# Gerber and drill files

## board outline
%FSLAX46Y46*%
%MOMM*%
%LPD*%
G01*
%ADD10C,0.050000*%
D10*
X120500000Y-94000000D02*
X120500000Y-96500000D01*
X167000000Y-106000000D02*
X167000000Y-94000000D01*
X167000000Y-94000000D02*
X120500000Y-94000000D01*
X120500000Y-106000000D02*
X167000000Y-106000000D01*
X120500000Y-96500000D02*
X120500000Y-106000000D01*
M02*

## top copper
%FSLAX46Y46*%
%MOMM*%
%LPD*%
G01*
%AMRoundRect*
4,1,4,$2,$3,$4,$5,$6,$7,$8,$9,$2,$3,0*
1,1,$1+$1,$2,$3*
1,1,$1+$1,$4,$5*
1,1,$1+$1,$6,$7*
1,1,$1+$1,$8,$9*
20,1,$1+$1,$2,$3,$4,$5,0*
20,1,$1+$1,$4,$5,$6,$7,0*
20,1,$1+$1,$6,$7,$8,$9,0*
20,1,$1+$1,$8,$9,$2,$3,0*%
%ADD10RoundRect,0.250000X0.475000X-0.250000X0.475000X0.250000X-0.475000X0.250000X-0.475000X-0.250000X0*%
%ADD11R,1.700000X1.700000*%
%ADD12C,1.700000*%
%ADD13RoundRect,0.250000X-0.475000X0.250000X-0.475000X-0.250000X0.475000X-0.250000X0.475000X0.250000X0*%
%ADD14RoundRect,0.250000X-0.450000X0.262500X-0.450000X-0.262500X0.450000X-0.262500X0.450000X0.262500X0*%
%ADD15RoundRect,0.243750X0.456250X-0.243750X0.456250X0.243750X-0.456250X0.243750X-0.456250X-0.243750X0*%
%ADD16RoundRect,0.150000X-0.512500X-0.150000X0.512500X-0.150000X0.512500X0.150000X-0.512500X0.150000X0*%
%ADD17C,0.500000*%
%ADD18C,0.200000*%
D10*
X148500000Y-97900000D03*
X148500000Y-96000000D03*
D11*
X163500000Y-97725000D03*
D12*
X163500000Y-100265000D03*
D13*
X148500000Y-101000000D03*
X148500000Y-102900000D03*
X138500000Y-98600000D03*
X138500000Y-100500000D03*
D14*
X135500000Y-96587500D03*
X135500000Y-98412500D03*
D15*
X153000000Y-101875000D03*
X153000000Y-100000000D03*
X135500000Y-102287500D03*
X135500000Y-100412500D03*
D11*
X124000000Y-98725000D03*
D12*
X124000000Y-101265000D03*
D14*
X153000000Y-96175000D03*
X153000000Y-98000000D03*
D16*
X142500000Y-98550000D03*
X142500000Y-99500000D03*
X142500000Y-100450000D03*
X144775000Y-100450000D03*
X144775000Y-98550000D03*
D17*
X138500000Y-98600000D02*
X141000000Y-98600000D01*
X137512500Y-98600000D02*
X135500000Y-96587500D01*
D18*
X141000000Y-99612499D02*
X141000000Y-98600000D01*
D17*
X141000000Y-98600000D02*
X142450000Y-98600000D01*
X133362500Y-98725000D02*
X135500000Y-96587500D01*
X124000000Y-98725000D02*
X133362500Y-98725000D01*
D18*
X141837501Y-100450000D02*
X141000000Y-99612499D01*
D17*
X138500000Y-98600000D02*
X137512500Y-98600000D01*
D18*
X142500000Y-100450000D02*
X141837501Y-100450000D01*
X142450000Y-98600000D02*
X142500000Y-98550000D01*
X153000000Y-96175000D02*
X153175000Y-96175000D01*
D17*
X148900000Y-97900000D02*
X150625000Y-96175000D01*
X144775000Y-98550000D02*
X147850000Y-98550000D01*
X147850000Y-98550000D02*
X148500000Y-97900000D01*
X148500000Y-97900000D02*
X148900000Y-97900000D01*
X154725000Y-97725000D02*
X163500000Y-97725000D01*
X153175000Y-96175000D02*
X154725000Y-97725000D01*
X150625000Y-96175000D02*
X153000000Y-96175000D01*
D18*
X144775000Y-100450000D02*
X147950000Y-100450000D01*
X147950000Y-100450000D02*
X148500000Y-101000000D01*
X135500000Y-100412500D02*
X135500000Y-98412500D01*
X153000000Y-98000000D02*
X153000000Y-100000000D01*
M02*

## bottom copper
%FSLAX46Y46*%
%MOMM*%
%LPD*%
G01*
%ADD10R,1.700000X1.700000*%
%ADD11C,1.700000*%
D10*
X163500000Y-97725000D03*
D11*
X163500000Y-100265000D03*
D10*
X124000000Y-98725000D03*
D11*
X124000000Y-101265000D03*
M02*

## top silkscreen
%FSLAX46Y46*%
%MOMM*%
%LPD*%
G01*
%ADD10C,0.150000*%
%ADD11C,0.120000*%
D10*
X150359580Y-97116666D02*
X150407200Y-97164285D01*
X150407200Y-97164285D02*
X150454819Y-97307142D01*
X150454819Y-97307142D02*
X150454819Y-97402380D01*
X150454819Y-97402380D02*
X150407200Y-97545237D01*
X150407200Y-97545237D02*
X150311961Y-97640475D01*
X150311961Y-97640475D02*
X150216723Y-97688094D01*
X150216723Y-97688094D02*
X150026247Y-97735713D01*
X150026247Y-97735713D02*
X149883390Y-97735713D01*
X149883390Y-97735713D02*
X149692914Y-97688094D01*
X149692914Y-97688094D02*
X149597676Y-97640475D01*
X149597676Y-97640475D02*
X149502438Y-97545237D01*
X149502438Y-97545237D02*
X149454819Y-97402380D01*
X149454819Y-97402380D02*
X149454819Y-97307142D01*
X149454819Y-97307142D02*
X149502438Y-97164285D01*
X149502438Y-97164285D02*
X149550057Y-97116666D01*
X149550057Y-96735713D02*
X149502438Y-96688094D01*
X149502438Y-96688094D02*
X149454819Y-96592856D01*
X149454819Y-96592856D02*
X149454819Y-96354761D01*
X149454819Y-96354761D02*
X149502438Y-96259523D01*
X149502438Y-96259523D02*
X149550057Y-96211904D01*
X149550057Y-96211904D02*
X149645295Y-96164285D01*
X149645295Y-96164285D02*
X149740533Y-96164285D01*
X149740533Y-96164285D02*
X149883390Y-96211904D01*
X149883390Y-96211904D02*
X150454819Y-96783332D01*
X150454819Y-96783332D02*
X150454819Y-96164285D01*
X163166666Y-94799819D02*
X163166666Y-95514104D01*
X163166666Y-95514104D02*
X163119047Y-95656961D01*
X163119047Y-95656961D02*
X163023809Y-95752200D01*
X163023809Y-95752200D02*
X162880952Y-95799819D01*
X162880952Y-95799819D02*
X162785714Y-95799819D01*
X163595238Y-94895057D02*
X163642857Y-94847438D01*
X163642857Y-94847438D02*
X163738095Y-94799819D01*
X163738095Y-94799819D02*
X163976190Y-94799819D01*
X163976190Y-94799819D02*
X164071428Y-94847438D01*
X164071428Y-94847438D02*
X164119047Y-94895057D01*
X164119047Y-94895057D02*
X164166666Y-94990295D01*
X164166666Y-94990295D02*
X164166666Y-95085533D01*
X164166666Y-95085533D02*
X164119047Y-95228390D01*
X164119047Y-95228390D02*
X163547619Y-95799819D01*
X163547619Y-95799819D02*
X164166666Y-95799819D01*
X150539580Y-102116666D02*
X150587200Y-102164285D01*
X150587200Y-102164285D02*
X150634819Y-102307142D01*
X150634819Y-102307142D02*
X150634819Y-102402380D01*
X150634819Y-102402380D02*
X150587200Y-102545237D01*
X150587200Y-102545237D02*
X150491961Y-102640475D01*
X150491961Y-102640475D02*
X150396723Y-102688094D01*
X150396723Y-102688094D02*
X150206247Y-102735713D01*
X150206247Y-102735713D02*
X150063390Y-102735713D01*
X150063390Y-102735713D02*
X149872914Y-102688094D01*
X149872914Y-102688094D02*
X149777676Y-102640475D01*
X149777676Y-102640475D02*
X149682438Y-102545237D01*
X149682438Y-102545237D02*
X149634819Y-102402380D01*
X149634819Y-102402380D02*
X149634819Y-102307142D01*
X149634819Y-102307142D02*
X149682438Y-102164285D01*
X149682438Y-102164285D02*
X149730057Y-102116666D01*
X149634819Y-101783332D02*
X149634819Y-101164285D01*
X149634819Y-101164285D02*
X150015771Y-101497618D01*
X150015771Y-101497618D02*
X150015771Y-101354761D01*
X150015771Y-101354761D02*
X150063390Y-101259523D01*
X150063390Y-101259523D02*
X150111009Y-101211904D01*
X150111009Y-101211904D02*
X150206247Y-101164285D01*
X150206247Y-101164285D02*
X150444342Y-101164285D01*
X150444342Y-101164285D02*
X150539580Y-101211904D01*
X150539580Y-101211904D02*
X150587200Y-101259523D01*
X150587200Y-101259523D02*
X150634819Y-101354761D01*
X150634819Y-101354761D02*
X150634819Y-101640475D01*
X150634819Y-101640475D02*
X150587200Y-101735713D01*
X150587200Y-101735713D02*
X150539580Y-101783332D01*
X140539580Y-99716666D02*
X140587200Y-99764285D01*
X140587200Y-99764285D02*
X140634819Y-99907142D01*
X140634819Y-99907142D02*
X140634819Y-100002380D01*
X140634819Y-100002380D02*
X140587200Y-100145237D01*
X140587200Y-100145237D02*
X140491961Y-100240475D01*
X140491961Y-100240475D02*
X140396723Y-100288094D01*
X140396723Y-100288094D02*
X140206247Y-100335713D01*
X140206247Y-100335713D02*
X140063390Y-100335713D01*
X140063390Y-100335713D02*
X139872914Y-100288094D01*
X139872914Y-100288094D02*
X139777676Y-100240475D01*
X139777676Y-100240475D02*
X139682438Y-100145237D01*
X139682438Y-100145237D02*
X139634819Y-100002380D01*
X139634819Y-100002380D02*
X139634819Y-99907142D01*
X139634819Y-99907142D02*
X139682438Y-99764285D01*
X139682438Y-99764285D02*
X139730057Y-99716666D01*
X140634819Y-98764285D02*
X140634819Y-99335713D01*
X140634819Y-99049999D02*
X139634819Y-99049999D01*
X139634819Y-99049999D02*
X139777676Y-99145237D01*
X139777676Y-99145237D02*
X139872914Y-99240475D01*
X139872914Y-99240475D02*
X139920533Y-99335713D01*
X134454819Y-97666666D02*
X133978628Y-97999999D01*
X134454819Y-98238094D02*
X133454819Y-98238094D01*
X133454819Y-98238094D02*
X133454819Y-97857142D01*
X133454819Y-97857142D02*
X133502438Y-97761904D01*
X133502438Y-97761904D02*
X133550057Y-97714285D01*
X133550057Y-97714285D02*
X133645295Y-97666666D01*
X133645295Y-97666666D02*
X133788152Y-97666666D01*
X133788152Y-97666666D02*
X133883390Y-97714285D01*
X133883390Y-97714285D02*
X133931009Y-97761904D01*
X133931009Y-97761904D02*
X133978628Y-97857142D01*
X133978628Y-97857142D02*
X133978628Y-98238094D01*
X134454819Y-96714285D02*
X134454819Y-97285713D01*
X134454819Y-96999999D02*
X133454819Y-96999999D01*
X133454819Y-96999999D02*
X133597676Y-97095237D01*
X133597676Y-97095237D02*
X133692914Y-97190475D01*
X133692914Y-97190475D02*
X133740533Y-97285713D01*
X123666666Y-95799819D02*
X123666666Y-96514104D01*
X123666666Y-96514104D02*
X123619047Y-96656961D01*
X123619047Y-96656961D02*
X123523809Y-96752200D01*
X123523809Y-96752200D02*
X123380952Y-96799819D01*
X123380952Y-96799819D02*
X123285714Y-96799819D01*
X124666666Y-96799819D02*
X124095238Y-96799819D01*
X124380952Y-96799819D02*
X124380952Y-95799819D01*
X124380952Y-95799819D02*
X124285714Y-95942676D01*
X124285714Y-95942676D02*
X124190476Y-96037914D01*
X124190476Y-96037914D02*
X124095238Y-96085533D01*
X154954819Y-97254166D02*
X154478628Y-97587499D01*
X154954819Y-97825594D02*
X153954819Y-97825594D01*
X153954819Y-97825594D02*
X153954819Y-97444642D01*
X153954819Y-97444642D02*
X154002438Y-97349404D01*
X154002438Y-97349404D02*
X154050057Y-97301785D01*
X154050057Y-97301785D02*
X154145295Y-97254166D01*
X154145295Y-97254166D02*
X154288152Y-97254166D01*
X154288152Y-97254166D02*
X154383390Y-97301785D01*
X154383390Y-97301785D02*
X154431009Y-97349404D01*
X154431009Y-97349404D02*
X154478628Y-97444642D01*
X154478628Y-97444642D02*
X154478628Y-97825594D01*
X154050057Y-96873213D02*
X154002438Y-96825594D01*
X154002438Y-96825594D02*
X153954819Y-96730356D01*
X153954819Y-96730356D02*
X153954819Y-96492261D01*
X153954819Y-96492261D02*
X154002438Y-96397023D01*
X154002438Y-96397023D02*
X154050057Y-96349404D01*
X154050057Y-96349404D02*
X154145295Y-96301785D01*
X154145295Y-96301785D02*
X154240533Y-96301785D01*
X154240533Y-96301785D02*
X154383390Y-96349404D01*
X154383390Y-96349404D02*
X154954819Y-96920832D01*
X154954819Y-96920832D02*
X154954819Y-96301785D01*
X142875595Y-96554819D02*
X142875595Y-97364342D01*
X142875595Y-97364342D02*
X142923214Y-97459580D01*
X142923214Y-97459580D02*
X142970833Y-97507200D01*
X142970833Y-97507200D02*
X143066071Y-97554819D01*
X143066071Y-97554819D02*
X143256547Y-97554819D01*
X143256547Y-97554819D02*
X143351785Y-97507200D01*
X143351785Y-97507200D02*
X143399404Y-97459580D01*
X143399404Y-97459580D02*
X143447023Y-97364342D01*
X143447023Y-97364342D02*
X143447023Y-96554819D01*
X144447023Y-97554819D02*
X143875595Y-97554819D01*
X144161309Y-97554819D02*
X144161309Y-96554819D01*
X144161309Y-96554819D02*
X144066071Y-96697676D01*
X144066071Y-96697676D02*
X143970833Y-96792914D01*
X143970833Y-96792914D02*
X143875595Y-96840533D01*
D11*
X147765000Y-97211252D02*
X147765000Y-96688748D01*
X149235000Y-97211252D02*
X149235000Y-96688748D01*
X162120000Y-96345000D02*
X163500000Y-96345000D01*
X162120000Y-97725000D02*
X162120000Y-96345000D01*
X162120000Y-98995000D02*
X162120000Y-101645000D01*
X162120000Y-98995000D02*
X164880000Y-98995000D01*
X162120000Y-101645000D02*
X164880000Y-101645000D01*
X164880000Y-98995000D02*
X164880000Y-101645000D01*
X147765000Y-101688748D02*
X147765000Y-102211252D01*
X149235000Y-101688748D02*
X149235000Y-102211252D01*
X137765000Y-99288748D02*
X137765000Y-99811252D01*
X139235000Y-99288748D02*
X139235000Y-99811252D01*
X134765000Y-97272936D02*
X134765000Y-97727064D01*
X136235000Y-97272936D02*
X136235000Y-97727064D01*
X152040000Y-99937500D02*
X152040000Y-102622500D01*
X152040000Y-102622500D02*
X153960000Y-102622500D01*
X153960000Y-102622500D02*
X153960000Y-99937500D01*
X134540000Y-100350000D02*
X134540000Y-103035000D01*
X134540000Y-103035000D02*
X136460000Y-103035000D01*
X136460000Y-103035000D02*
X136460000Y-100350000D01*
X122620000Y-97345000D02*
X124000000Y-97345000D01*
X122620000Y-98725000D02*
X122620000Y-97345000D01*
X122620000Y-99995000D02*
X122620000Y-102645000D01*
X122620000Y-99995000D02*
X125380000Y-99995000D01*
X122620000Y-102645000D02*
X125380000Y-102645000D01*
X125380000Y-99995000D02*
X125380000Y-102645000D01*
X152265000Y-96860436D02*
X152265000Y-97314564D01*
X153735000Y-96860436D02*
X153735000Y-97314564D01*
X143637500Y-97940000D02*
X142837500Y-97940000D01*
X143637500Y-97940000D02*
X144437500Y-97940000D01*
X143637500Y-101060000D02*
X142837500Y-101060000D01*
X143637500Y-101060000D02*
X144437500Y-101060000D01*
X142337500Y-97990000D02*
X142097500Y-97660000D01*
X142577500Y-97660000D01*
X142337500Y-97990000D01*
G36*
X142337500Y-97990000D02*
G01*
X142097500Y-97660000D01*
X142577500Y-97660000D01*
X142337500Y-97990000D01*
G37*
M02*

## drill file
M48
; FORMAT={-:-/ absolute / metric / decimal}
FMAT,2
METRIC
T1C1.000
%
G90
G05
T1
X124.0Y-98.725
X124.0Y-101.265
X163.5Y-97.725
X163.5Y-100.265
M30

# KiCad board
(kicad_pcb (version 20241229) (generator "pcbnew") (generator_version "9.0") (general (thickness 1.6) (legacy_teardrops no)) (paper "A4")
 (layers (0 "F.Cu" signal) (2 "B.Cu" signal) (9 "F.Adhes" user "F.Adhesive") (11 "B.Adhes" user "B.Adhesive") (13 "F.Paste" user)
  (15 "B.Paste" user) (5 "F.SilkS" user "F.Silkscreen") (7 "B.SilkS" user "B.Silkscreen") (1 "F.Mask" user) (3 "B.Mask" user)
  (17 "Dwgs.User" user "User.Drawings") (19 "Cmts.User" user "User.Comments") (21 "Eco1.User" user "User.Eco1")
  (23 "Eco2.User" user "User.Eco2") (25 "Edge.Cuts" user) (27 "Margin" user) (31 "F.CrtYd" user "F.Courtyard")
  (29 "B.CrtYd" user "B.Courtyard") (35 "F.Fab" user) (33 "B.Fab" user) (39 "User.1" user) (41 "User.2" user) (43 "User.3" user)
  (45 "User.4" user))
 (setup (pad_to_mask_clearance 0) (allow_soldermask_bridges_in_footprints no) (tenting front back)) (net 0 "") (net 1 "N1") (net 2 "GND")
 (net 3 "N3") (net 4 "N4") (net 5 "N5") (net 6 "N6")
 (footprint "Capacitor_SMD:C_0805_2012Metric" (layer "F.Cu") (at 148.5 96.95 90)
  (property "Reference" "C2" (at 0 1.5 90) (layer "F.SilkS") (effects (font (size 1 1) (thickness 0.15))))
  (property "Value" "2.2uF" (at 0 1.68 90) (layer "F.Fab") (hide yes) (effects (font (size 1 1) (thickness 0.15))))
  (fp_line (start -0.261252 -0.735) (end 0.261252 -0.735) (stroke (width 0.12) (type solid)) (layer "F.SilkS"))
  (fp_line (start -0.261252 0.735) (end 0.261252 0.735) (stroke (width 0.12) (type solid)) (layer "F.SilkS"))
  (pad "1" smd roundrect (at -0.95 0 90) (size 1 1.45) (layers "F.Cu" "F.Mask" "F.Paste") (roundrect_rratio 0.25) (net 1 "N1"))
  (pad "2" smd roundrect (at 0.95 0 90) (size 1 1.45) (layers "F.Cu" "F.Mask" "F.Paste") (roundrect_rratio 0.25) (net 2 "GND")))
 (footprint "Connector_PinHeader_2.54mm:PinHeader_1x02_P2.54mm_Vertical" (layer "F.Cu") (at 163.5 97.725)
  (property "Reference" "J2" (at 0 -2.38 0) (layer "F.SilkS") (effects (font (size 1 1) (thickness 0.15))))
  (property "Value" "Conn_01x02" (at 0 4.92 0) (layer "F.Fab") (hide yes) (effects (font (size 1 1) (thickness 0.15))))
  (fp_line (start -1.38 -1.38) (end 0 -1.38) (stroke (width 0.12) (type solid)) (layer "F.SilkS"))
  (fp_line (start -1.38 0) (end -1.38 -1.38) (stroke (width 0.12) (type solid)) (layer "F.SilkS"))
  (fp_line (start -1.38 1.27) (end -1.38 3.92) (stroke (width 0.12) (type solid)) (layer "F.SilkS"))
  (fp_line (start -1.38 1.27) (end 1.38 1.27) (stroke (width 0.12) (type solid)) (layer "F.SilkS"))
  (fp_line (start -1.38 3.92) (end 1.38 3.92) (stroke (width 0.12) (type solid)) (layer "F.SilkS"))
  (fp_line (start 1.38 1.27) (end 1.38 3.92) (stroke (width 0.12) (type solid)) (layer "F.SilkS"))
  (pad "1" thru_hole rect (at 0 0) (size 1.7 1.7) (drill 1) (layers "*.Cu" "*.Mask") (remove_unused_layers no) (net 1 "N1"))
  (pad "2" thru_hole circle (at 0 2.54) (size 1.7 1.7) (drill 1) (layers "*.Cu" "*.Mask") (remove_unused_layers no) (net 2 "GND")))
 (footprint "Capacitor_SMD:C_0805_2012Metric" (layer "F.Cu") (at 148.5 101.95 -90)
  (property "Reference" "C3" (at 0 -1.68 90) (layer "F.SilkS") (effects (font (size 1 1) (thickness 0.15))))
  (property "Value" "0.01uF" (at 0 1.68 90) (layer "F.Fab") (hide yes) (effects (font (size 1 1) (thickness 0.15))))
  (fp_line (start -0.261252 0.735) (end 0.261252 0.735) (stroke (width 0.12) (type solid)) (layer "F.SilkS"))
  (fp_line (start -0.261252 -0.735) (end 0.261252 -0.735) (stroke (width 0.12) (type solid)) (layer "F.SilkS"))
  (pad "1" smd roundrect (at -0.95 0 270) (size 1 1.45) (layers "F.Cu" "F.Mask" "F.Paste") (roundrect_rratio 0.25) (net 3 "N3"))
  (pad "2" smd roundrect (at 0.95 0 270) (size 1 1.45) (layers "F.Cu" "F.Mask" "F.Paste") (roundrect_rratio 0.25) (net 2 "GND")))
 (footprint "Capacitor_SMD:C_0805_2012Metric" (layer "F.Cu") (at 138.5 99.55 -90)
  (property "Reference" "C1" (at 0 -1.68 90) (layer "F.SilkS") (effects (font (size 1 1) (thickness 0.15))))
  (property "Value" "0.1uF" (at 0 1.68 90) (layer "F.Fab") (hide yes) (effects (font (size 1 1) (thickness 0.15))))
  (fp_line (start -0.261252 0.735) (end 0.261252 0.735) (stroke (width 0.12) (type solid)) (layer "F.SilkS"))
  (fp_line (start -0.261252 -0.735) (end 0.261252 -0.735) (stroke (width 0.12) (type solid)) (layer "F.SilkS"))
  (pad "1" smd roundrect (at -0.95 0 270) (size 1 1.45) (layers "F.Cu" "F.Mask" "F.Paste") (roundrect_rratio 0.25) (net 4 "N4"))
  (pad "2" smd roundrect (at 0.95 0 270) (size 1 1.45) (layers "F.Cu" "F.Mask" "F.Paste") (roundrect_rratio 0.25) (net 2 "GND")))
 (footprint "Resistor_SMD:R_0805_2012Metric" (layer "F.Cu") (at 135.5 97.5 -90)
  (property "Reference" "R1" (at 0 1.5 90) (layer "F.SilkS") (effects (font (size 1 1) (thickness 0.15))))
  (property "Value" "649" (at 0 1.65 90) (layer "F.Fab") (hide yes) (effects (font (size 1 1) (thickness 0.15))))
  (fp_line (start -0.227064 0.735) (end 0.227064 0.735) (stroke (width 0.12) (type solid)) (layer "F.SilkS"))
  (fp_line (start -0.227064 -0.735) (end 0.227064 -0.735) (stroke (width 0.12) (type solid)) (layer "F.SilkS"))
  (pad "1" smd roundrect (at -0.9125 0 270) (size 1.025 1.4) (layers "F.Cu" "F.Mask" "F.Paste") (roundrect_rratio 0.243902) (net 4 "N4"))
  (pad "2" smd roundrect (at 0.9125 0 270) (size 1.025 1.4) (layers "F.Cu" "F.Mask" "F.Paste") (roundrect_rratio 0.243902) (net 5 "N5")))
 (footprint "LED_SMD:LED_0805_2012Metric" (layer "F.Cu") (at 153 100.9375 90)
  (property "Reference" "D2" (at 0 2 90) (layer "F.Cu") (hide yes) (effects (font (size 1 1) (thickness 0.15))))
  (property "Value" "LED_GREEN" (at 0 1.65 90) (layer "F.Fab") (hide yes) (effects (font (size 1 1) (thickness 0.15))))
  (fp_line (start 1 -0.96) (end -1.685 -0.96) (stroke (width 0.12) (type solid)) (layer "F.SilkS"))
  (fp_line (start -1.685 -0.96) (end -1.685 0.96) (stroke (width 0.12) (type solid)) (layer "F.SilkS"))
  (fp_line (start -1.685 0.96) (end 1 0.96) (stroke (width 0.12) (type solid)) (layer "F.SilkS"))
  (pad "1" smd roundrect (at -0.9375 0 90) (size 0.975 1.4) (layers "F.Cu" "F.Mask" "F.Paste") (roundrect_rratio 0.25) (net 2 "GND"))
  (pad "2" smd roundrect (at 0.9375 0 90) (size 0.975 1.4) (layers "F.Cu" "F.Mask" "F.Paste") (roundrect_rratio 0.25) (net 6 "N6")))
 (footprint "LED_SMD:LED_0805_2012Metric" (layer "F.Cu") (at 135.5 101.35 90)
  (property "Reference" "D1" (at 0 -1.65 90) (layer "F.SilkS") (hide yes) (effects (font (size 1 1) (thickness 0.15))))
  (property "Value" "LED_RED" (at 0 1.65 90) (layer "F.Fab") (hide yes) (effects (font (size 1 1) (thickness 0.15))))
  (fp_line (start 1 -0.96) (end -1.685 -0.96) (stroke (width 0.12) (type solid)) (layer "F.SilkS"))
  (fp_line (start -1.685 -0.96) (end -1.685 0.96) (stroke (width 0.12) (type solid)) (layer "F.SilkS"))
  (fp_line (start -1.685 0.96) (end 1 0.96) (stroke (width 0.12) (type solid)) (layer "F.SilkS"))
  (pad "1" smd roundrect (at -0.9375 0 90) (size 0.975 1.4) (layers "F.Cu" "F.Mask" "F.Paste") (roundrect_rratio 0.25) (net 2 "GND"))
  (pad "2" smd roundrect (at 0.9375 0 90) (size 0.975 1.4) (layers "F.Cu" "F.Mask" "F.Paste") (roundrect_rratio 0.25) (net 5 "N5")))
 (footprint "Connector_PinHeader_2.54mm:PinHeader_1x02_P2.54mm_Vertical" (layer "F.Cu") (at 124 98.725)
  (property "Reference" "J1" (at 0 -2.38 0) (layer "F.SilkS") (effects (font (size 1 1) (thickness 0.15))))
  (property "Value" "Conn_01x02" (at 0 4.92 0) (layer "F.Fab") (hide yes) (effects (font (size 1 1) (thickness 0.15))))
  (fp_line (start -1.38 -1.38) (end 0 -1.38) (stroke (width 0.12) (type solid)) (layer "F.SilkS"))
  (fp_line (start -1.38 0) (end -1.38 -1.38) (stroke (width 0.12) (type solid)) (layer "F.SilkS"))
  (fp_line (start -1.38 1.27) (end -1.38 3.92) (stroke (width 0.12) (type solid)) (layer "F.SilkS"))
  (fp_line (start -1.38 1.27) (end 1.38 1.27) (stroke (width 0.12) (type solid)) (layer "F.SilkS"))
  (fp_line (start -1.38 3.92) (end 1.38 3.92) (stroke (width 0.12) (type solid)) (layer "F.SilkS"))
  (fp_line (start 1.38 1.27) (end 1.38 3.92) (stroke (width 0.12) (type solid)) (layer "F.SilkS"))
  (pad "1" thru_hole rect (at 0 0) (size 1.7 1.7) (drill 1) (layers "*.Cu" "*.Mask") (remove_unused_layers no) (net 4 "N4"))
  (pad "2" thru_hole circle (at 0 2.54) (size 1.7 1.7) (drill 1) (layers "*.Cu" "*.Mask") (remove_unused_layers no) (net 2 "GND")))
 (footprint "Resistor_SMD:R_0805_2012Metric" (layer "F.Cu") (at 153 97.0875 -90)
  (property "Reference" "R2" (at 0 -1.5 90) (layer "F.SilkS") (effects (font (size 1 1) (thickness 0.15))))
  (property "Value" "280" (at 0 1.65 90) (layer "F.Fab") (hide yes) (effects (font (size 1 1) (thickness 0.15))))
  (fp_line (start -0.227064 0.735) (end 0.227064 0.735) (stroke (width 0.12) (type solid)) (layer "F.SilkS"))
  (fp_line (start -0.227064 -0.735) (end 0.227064 -0.735) (stroke (width 0.12) (type solid)) (layer "F.SilkS"))
  (pad "1" smd roundrect (at -0.9125 0 270) (size 1.025 1.4) (layers "F.Cu" "F.Mask" "F.Paste") (roundrect_rratio 0.243902) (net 1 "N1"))
  (pad "2" smd roundrect (at 0.9125 0 270) (size 1.025 1.4) (layers "F.Cu" "F.Mask" "F.Paste") (roundrect_rratio 0.243902) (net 6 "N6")))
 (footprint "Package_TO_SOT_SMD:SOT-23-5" (layer "F.Cu") (at 143.6375 99.5)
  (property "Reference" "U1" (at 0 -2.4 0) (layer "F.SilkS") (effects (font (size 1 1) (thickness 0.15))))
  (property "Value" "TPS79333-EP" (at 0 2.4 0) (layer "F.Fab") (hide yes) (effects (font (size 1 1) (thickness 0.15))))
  (fp_line (start 0 -1.56) (end -0.8 -1.56) (stroke (width 0.12) (type solid)) (layer "F.SilkS"))
  (fp_line (start 0 -1.56) (end 0.8 -1.56) (stroke (width 0.12) (type solid)) (layer "F.SilkS"))
  (fp_line (start 0 1.56) (end -0.8 1.56) (stroke (width 0.12) (type solid)) (layer "F.SilkS"))
  (fp_line (start 0 1.56) (end 0.8 1.56) (stroke (width 0.12) (type solid)) (layer "F.SilkS"))
  (fp_poly (pts (xy -1.3 -1.51) (xy -1.54 -1.84) (xy -1.06 -1.84)) (stroke (width 0.12) (type solid)) (fill yes) (layer "F.SilkS"))
  (pad "1" smd roundrect (at -1.1375 -0.95) (size 1.325 0.6) (layers "F.Cu" "F.Mask" "F.Paste") (roundrect_rratio 0.25) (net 4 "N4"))
  (pad "2" smd roundrect (at -1.1375 0) (size 1.325 0.6) (layers "F.Cu" "F.Mask" "F.Paste") (roundrect_rratio 0.25) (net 2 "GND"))
  (pad "3" smd roundrect (at -1.1375 0.95) (size 1.325 0.6) (layers "F.Cu" "F.Mask" "F.Paste") (roundrect_rratio 0.25) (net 4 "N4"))
  (pad "4" smd roundrect (at 1.1375 0.95) (size 1.325 0.6) (layers "F.Cu" "F.Mask" "F.Paste") (roundrect_rratio 0.25) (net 3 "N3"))
  (pad "5" smd roundrect (at 1.1375 -0.95) (size 1.325 0.6) (layers "F.Cu" "F.Mask" "F.Paste") (roundrect_rratio 0.25) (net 1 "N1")))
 (gr_line (start 120.5 94) (end 120.5 96.5) (stroke (width 0.05) (type default)) (layer "Edge.Cuts"))
 (gr_line (start 167 106) (end 167 94) (stroke (width 0.05) (type default)) (layer "Edge.Cuts"))
 (gr_line (start 167 94) (end 120.5 94) (stroke (width 0.05) (type default)) (layer "Edge.Cuts"))
 (gr_line (start 120.5 106) (end 167 106) (stroke (width 0.05) (type default)) (layer "Edge.Cuts"))
 (gr_line (start 120.5 96.5) (end 120.5 106) (stroke (width 0.05) (type default)) (layer "Edge.Cuts"))
 (segment (start 138.5 98.6) (end 141 98.6) (width 0.5) (layer "F.Cu") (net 4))
 (segment (start 137.5125 98.6) (end 135.5 96.5875) (width 0.5) (layer "F.Cu") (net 4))
 (segment (start 141 99.612499) (end 141 98.6) (width 0.2) (layer "F.Cu") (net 4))
 (segment (start 141 98.6) (end 142.45 98.6) (width 0.5) (layer "F.Cu") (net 4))
 (segment (start 133.3625 98.725) (end 135.5 96.5875) (width 0.5) (layer "F.Cu") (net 4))
 (segment (start 124 98.725) (end 133.3625 98.725) (width 0.5) (layer "F.Cu") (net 4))
 (segment (start 141.837501 100.45) (end 141 99.612499) (width 0.2) (layer "F.Cu") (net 4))
 (segment (start 138.5 98.6) (end 137.5125 98.6) (width 0.5) (layer "F.Cu") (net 4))
 (segment (start 142.5 100.45) (end 141.837501 100.45) (width 0.2) (layer "F.Cu") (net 4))
 (segment (start 142.45 98.6) (end 142.5 98.55) (width 0.2) (layer "F.Cu") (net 4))
 (segment (start 153 96.175) (end 153.175 96.175) (width 0.2) (layer "F.Cu") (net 1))
 (segment (start 148.9 97.9) (end 150.625 96.175) (width 0.5) (layer "F.Cu") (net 1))
 (segment (start 144.775 98.55) (end 147.85 98.55) (width 0.5) (layer "F.Cu") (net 1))
 (segment (start 147.85 98.55) (end 148.5 97.9) (width 0.5) (layer "F.Cu") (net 1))
 (segment (start 148.5 97.9) (end 148.9 97.9) (width 0.5) (layer "F.Cu") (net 1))
 (segment (start 154.725 97.725) (end 163.5 97.725) (width 0.5) (layer "F.Cu") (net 1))
 (segment (start 153.175 96.175) (end 154.725 97.725) (width 0.5) (layer "F.Cu") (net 1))
 (segment (start 150.625 96.175) (end 153 96.175) (width 0.5) (layer "F.Cu") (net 1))
 (segment (start 144.775 100.45) (end 147.95 100.45) (width 0.2) (layer "F.Cu") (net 3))
 (segment (start 147.95 100.45) (end 148.5 101) (width 0.2) (layer "F.Cu") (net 3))
 (segment (start 135.5 100.4125) (end 135.5 98.4125) (width 0.2) (layer "F.Cu") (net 5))
 (segment (start 153 98) (end 153 100) (width 0.2) (layer "F.Cu") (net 6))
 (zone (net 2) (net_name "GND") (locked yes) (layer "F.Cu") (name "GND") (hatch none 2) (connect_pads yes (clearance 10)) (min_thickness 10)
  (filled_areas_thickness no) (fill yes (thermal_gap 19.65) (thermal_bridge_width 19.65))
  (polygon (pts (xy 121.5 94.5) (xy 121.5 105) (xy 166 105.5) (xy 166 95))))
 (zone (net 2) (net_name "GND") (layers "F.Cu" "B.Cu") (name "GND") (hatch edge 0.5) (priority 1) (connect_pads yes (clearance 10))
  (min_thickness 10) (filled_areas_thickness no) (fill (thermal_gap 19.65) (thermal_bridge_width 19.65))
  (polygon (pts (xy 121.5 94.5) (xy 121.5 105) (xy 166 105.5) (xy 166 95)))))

